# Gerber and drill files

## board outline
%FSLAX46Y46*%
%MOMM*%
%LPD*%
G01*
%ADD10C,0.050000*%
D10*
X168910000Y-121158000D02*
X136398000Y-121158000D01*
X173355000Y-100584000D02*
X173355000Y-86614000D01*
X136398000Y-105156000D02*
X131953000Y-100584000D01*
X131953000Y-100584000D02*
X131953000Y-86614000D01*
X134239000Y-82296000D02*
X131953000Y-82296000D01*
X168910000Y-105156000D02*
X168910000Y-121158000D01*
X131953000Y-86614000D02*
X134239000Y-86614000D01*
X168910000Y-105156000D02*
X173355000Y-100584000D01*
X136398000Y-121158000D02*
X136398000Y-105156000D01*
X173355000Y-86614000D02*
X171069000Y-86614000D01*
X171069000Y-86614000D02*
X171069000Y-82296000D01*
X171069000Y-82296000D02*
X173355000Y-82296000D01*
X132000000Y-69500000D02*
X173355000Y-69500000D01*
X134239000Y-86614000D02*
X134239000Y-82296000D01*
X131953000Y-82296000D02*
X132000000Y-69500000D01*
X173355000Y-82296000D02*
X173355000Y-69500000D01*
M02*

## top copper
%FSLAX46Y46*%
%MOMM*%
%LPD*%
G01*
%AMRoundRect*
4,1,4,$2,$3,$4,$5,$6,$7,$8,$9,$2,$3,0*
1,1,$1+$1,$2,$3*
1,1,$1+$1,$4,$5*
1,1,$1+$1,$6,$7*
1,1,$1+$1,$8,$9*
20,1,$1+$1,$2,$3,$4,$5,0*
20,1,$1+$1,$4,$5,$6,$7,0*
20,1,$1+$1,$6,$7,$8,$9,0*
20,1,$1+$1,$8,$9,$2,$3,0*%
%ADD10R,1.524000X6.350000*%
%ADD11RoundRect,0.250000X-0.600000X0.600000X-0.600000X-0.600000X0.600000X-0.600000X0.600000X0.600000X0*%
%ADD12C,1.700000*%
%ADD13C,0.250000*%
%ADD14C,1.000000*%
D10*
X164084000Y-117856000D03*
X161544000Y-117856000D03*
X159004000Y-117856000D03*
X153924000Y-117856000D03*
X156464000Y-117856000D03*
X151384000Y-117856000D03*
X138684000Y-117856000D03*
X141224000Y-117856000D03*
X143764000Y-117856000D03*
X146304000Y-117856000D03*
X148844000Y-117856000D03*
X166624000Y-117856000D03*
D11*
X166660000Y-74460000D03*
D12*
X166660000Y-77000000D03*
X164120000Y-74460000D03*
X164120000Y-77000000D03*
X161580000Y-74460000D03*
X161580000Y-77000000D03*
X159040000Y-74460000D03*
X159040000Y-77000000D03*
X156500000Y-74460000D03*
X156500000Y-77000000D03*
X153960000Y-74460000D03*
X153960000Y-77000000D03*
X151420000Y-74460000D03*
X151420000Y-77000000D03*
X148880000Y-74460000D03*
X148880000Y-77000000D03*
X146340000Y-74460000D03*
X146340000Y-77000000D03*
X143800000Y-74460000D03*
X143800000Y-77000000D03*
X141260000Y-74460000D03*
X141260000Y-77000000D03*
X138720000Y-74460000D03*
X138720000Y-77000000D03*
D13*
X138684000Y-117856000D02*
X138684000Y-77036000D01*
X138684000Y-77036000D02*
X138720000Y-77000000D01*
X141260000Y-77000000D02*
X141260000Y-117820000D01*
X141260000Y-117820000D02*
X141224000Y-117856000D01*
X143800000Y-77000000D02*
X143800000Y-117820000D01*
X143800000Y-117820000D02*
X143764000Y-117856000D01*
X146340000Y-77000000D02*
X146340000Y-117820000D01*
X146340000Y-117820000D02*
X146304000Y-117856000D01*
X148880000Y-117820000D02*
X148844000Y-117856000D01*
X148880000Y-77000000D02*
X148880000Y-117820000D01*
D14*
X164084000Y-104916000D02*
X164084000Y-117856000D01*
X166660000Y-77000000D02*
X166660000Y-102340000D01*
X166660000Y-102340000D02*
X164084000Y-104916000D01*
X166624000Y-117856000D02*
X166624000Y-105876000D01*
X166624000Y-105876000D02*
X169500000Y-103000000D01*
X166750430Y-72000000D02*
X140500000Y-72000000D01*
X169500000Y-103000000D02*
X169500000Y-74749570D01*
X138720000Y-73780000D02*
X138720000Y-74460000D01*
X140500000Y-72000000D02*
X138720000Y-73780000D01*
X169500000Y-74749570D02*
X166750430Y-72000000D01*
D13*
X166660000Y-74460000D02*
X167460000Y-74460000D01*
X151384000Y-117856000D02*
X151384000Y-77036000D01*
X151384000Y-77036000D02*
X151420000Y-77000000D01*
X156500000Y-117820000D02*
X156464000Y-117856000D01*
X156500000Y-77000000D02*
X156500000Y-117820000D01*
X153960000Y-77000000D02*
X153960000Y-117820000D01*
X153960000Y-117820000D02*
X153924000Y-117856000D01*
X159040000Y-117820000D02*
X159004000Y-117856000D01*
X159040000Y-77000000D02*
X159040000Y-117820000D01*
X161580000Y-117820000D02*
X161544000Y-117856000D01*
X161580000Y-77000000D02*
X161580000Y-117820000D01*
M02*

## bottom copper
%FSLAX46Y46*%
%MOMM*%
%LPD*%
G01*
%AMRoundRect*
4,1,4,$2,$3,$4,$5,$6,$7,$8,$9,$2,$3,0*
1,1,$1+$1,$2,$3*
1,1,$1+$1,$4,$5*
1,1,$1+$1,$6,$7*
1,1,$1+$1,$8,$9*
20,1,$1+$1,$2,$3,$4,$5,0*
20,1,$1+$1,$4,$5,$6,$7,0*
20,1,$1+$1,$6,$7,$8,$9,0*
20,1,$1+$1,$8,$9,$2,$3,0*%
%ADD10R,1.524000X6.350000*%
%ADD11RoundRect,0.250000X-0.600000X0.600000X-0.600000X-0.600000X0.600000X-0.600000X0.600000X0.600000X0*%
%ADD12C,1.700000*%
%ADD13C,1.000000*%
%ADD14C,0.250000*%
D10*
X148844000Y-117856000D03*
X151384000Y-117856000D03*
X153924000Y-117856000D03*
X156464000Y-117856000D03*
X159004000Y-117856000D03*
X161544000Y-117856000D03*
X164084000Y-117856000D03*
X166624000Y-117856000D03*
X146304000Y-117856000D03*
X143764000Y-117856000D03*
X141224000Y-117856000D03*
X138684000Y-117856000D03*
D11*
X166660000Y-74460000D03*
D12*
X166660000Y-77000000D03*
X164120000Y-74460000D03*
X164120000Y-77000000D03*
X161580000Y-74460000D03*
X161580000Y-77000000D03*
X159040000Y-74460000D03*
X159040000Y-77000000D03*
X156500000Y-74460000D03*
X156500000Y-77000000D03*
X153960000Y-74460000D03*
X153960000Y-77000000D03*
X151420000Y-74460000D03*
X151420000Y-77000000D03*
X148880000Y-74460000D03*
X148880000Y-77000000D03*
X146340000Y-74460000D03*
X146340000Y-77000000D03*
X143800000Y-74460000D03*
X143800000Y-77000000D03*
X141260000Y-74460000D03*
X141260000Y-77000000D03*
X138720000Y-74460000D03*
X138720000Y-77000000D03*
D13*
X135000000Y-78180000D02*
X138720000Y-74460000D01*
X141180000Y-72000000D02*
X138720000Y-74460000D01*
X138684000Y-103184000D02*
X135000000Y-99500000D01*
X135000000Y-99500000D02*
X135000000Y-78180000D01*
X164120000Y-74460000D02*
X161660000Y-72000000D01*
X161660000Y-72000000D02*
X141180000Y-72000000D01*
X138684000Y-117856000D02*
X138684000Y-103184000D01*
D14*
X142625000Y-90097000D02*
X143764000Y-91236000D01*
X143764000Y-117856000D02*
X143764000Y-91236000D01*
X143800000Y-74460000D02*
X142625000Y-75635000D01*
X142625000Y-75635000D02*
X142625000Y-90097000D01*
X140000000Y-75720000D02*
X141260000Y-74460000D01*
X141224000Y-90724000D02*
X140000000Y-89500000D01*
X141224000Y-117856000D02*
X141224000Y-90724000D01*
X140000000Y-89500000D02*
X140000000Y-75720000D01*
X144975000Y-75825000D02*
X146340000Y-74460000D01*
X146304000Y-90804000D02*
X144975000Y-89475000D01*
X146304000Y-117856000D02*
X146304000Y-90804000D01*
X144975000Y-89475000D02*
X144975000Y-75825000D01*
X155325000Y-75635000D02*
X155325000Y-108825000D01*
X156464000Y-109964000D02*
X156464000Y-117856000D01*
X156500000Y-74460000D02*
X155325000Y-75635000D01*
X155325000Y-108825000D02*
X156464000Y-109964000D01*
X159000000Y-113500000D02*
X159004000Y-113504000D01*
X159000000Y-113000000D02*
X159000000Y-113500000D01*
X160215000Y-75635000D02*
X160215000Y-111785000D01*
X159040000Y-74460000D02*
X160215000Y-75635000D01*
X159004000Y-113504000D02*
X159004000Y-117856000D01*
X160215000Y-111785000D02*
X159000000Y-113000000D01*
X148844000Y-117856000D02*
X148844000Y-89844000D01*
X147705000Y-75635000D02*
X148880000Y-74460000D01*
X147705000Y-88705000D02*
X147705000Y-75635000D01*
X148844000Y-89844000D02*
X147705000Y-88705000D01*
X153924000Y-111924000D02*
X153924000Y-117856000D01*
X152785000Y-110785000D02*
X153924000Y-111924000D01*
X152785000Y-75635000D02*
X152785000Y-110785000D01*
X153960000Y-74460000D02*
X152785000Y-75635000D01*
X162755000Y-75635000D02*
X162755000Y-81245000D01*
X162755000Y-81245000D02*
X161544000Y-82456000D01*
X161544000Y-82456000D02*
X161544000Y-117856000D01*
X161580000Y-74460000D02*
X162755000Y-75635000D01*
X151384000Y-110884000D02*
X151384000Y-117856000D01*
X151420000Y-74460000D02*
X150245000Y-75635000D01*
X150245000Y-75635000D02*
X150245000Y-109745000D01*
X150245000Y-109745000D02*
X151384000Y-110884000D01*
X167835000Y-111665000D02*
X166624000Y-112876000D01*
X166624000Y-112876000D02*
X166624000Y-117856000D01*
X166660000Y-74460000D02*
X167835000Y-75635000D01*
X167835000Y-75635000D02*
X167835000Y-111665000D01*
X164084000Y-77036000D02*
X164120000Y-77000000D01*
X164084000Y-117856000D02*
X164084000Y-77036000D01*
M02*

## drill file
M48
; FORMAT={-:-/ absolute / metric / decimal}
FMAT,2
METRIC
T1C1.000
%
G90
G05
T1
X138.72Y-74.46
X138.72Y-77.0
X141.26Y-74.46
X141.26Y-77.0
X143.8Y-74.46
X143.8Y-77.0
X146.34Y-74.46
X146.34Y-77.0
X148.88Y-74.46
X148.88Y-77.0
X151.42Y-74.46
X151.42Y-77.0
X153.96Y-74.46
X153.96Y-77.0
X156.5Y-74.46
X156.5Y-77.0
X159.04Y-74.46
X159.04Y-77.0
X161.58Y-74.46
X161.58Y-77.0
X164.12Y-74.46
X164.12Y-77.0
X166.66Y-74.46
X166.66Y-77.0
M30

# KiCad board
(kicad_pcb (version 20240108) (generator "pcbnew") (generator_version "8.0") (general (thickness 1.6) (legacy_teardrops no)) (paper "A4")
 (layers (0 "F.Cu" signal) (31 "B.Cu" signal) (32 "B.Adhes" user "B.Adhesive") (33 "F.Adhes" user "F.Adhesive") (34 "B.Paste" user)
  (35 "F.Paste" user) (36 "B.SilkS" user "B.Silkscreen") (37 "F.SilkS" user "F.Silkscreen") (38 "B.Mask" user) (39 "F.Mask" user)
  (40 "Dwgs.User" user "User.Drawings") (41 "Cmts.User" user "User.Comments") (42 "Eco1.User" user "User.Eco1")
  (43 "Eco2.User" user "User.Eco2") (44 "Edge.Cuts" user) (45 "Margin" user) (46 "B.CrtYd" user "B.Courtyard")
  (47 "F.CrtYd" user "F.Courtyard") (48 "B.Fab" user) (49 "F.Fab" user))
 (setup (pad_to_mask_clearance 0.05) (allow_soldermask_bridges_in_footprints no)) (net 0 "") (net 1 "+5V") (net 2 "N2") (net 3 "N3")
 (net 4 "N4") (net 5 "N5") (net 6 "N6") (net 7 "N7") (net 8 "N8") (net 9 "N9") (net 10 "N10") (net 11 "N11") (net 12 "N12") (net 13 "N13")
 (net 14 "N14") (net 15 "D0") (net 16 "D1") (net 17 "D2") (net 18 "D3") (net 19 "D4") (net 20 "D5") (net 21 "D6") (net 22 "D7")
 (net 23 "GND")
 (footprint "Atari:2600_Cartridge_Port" (layer "F.Cu") (at 138.176 114.808)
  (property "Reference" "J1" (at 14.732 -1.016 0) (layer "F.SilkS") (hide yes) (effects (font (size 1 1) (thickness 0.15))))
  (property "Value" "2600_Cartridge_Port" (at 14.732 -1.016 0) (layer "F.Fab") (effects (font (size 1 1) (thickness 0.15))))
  (pad "+5V" connect rect (at 25.908 3.048) (size 1.524 6.35) (layers "F.Cu" "F.Mask") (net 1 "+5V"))
  (pad "A0" connect rect (at 10.668 3.048) (size 1.524 6.35) (layers "B.Cu" "B.Mask") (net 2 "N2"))
  (pad "A1" connect rect (at 13.208 3.048) (size 1.524 6.35) (layers "B.Cu" "B.Mask") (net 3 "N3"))
  (pad "A2" connect rect (at 15.748 3.048) (size 1.524 6.35) (layers "B.Cu" "B.Mask") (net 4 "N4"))
  (pad "A3" connect rect (at 18.288 3.048) (size 1.524 6.35) (layers "B.Cu" "B.Mask") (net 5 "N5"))
  (pad "A4" connect rect (at 20.828 3.048) (size 1.524 6.35) (layers "B.Cu" "B.Mask") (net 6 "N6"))
  (pad "A5" connect rect (at 23.368 3.048) (size 1.524 6.35) (layers "B.Cu" "B.Mask") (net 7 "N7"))
  (pad "A6" connect rect (at 25.908 3.048) (size 1.524 6.35) (layers "B.Cu" "B.Mask") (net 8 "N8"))
  (pad "A7" connect rect (at 28.448 3.048) (size 1.524 6.35) (layers "B.Cu" "B.Mask") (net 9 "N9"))
  (pad "A8" connect rect (at 23.368 3.048) (size 1.524 6.35) (layers "F.Cu" "F.Mask") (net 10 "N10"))
  (pad "A9" connect rect (at 20.828 3.048) (size 1.524 6.35) (layers "F.Cu" "F.Mask") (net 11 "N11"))
  (pad "A10" connect rect (at 15.748 3.048) (size 1.524 6.35) (layers "F.Cu" "F.Mask") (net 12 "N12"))
  (pad "A11" connect rect (at 18.288 3.048) (size 1.524 6.35) (layers "F.Cu" "F.Mask") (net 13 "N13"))
  (pad "A12" connect rect (at 13.208 3.048) (size 1.524 6.35) (layers "F.Cu" "F.Mask") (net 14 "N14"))
  (pad "D0" connect rect (at 8.128 3.048) (size 1.524 6.35) (layers "B.Cu" "B.Mask") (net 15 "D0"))
  (pad "D1" connect rect (at 5.588 3.048) (size 1.524 6.35) (layers "B.Cu" "B.Mask") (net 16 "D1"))
  (pad "D2" connect rect (at 3.048 3.048) (size 1.524 6.35) (layers "B.Cu" "B.Mask") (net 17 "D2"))
  (pad "D3" connect rect (at 0.508 3.048) (size 1.524 6.35) (layers "F.Cu" "F.Mask") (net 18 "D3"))
  (pad "D4" connect rect (at 3.048 3.048) (size 1.524 6.35) (layers "F.Cu" "F.Mask") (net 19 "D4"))
  (pad "D5" connect rect (at 5.588 3.048) (size 1.524 6.35) (layers "F.Cu" "F.Mask") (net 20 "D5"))
  (pad "D6" connect rect (at 8.128 3.048) (size 1.524 6.35) (layers "F.Cu" "F.Mask") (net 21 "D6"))
  (pad "D7" connect rect (at 10.668 3.048) (size 1.524 6.35) (layers "F.Cu" "F.Mask") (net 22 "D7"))
  (pad "GND" connect rect (at 0.508 3.048) (size 1.524 6.35) (layers "B.Cu" "B.Mask") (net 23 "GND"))
  (pad "SGND" connect rect (at 28.448 3.048) (size 1.524 6.35) (layers "F.Cu" "F.Mask") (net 23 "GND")))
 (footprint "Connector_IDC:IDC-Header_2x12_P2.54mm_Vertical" (layer "F.Cu") (at 166.66 74.46 -90)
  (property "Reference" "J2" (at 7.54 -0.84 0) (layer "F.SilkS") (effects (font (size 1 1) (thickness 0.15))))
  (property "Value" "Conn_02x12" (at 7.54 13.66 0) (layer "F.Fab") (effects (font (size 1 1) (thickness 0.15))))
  (pad "1" thru_hole roundrect (at 0 0 270) (size 1.7 1.7) (drill 1) (layers "*.Cu" "*.Mask") (remove_unused_layers no)
   (roundrect_rratio 0.147059) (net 9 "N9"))
  (pad "2" thru_hole circle (at 2.54 0 270) (size 1.7 1.7) (drill 1) (layers "*.Cu" "*.Mask") (remove_unused_layers no) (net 1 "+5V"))
  (pad "3" thru_hole circle (at 0 2.54 270) (size 1.7 1.7) (drill 1) (layers "*.Cu" "*.Mask") (remove_unused_layers no) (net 23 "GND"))
  (pad "4" thru_hole circle (at 2.54 2.54 270) (size 1.7 1.7) (drill 1) (layers "*.Cu" "*.Mask") (remove_unused_layers no) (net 8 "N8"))
  (pad "5" thru_hole circle (at 0 5.08 270) (size 1.7 1.7) (drill 1) (layers "*.Cu" "*.Mask") (remove_unused_layers no) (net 7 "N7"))
  (pad "6" thru_hole circle (at 2.54 5.08 270) (size 1.7 1.7) (drill 1) (layers "*.Cu" "*.Mask") (remove_unused_layers no) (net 10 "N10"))
  (pad "7" thru_hole circle (at 0 7.62 270) (size 1.7 1.7) (drill 1) (layers "*.Cu" "*.Mask") (remove_unused_layers no) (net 6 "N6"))
  (pad "8" thru_hole circle (at 2.54 7.62 270) (size 1.7 1.7) (drill 1) (layers "*.Cu" "*.Mask") (remove_unused_layers no) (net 11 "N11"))
  (pad "9" thru_hole circle (at 0 10.16 270) (size 1.7 1.7) (drill 1) (layers "*.Cu" "*.Mask") (remove_unused_layers no) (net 5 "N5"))
  (pad "10" thru_hole circle (at 2.54 10.16 270) (size 1.7 1.7) (drill 1) (layers "*.Cu" "*.Mask") (remove_unused_layers no) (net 13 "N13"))
  (pad "11" thru_hole circle (at 0 12.7 270) (size 1.7 1.7) (drill 1) (layers "*.Cu" "*.Mask") (remove_unused_layers no) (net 4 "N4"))
  (pad "12" thru_hole circle (at 2.54 12.7 270) (size 1.7 1.7) (drill 1) (layers "*.Cu" "*.Mask") (remove_unused_layers no) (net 12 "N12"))
  (pad "13" thru_hole circle (at 0 15.24 270) (size 1.7 1.7) (drill 1) (layers "*.Cu" "*.Mask") (remove_unused_layers no) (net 3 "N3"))
  (pad "14" thru_hole circle (at 2.54 15.24 270) (size 1.7 1.7) (drill 1) (layers "*.Cu" "*.Mask") (remove_unused_layers no) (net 14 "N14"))
  (pad "15" thru_hole circle (at 0 17.78 270) (size 1.7 1.7) (drill 1) (layers "*.Cu" "*.Mask") (remove_unused_layers no) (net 2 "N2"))
  (pad "16" thru_hole circle (at 2.54 17.78 270) (size 1.7 1.7) (drill 1) (layers "*.Cu" "*.Mask") (remove_unused_layers no) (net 22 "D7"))
  (pad "17" thru_hole circle (at 0 20.32 270) (size 1.7 1.7) (drill 1) (layers "*.Cu" "*.Mask") (remove_unused_layers no) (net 15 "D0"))
  (pad "18" thru_hole circle (at 2.54 20.32 270) (size 1.7 1.7) (drill 1) (layers "*.Cu" "*.Mask") (remove_unused_layers no) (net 21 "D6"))
  (pad "19" thru_hole circle (at 0 22.86 270) (size 1.7 1.7) (drill 1) (layers "*.Cu" "*.Mask") (remove_unused_layers no) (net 16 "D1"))
  (pad "20" thru_hole circle (at 2.54 22.86 270) (size 1.7 1.7) (drill 1) (layers "*.Cu" "*.Mask") (remove_unused_layers no) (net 20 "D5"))
  (pad "21" thru_hole circle (at 0 25.4 270) (size 1.7 1.7) (drill 1) (layers "*.Cu" "*.Mask") (remove_unused_layers no) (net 17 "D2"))
  (pad "22" thru_hole circle (at 2.54 25.4 270) (size 1.7 1.7) (drill 1) (layers "*.Cu" "*.Mask") (remove_unused_layers no) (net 19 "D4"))
  (pad "23" thru_hole circle (at 0 27.94 270) (size 1.7 1.7) (drill 1) (layers "*.Cu" "*.Mask") (remove_unused_layers no) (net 23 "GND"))
  (pad "24" thru_hole circle (at 2.54 27.94 270) (size 1.7 1.7) (drill 1) (layers "*.Cu" "*.Mask") (remove_unused_layers no) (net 18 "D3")))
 (gr_line (start 168.91 121.158) (end 136.398 121.158) (stroke (width 0.05) (type solid)) (layer "Edge.Cuts"))
 (gr_line (start 173.355 100.584) (end 173.355 86.614) (stroke (width 0.05) (type solid)) (layer "Edge.Cuts"))
 (gr_line (start 136.398 105.156) (end 131.953 100.584) (stroke (width 0.05) (type solid)) (layer "Edge.Cuts"))
 (gr_line (start 131.953 100.584) (end 131.953 86.614) (stroke (width 0.05) (type solid)) (layer "Edge.Cuts"))
 (gr_line (start 134.239 82.296) (end 131.953 82.296) (stroke (width 0.05) (type solid)) (layer "Edge.Cuts"))
 (gr_line (start 168.91 105.156) (end 168.91 121.158) (stroke (width 0.05) (type solid)) (layer "Edge.Cuts"))
 (gr_line (start 131.953 86.614) (end 134.239 86.614) (stroke (width 0.05) (type solid)) (layer "Edge.Cuts"))
 (gr_line (start 168.91 105.156) (end 173.355 100.584) (stroke (width 0.05) (type solid)) (layer "Edge.Cuts"))
 (gr_line (start 136.398 121.158) (end 136.398 105.156) (stroke (width 0.05) (type solid)) (layer "Edge.Cuts"))
 (gr_line (start 173.355 86.614) (end 171.069 86.614) (stroke (width 0.05) (type solid)) (layer "Edge.Cuts"))
 (gr_line (start 171.069 86.614) (end 171.069 82.296) (stroke (width 0.05) (type solid)) (layer "Edge.Cuts"))
 (gr_line (start 171.069 82.296) (end 173.355 82.296) (stroke (width 0.05) (type solid)) (layer "Edge.Cuts"))
 (gr_line (start 132 69.5) (end 173.355 69.5) (stroke (width 0.05) (type solid)) (layer "Edge.Cuts"))
 (gr_line (start 134.239 86.614) (end 134.239 82.296) (stroke (width 0.05) (type solid)) (layer "Edge.Cuts"))
 (gr_line (start 131.953 82.296) (end 132 69.5) (stroke (width 0.05) (type solid)) (layer "Edge.Cuts"))
 (gr_line (start 173.355 82.296) (end 173.355 69.5) (stroke (width 0.05) (type solid)) (layer "Edge.Cuts"))
 (segment (start 138.684 117.856) (end 138.684 77.036) (width 0.25) (layer "F.Cu") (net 18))
 (segment (start 138.684 77.036) (end 138.72 77) (width 0.25) (layer "F.Cu") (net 18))
 (segment (start 141.26 77) (end 141.26 117.82) (width 0.25) (layer "F.Cu") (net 19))
 (segment (start 141.26 117.82) (end 141.224 117.856) (width 0.25) (layer "F.Cu") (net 19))
 (segment (start 143.8 77) (end 143.8 117.82) (width 0.25) (layer "F.Cu") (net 20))
 (segment (start 143.8 117.82) (end 143.764 117.856) (width 0.25) (layer "F.Cu") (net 20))
 (segment (start 146.34 77) (end 146.34 117.82) (width 0.25) (layer "F.Cu") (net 21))
 (segment (start 146.34 117.82) (end 146.304 117.856) (width 0.25) (layer "F.Cu") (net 21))
 (segment (start 148.88 117.82) (end 148.844 117.856) (width 0.25) (layer "F.Cu") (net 22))
 (segment (start 148.88 77) (end 148.88 117.82) (width 0.25) (layer "F.Cu") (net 22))
 (segment (start 164.084 104.916) (end 164.084 117.856) (width 1) (layer "F.Cu") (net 1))
 (segment (start 166.66 77) (end 166.66 102.34) (width 1) (layer "F.Cu") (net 1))
 (segment (start 166.66 102.34) (end 164.084 104.916) (width 1) (layer "F.Cu") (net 1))
 (segment (start 166.624 117.856) (end 166.624 105.876) (width 1) (layer "F.Cu") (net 23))
 (segment (start 166.624 105.876) (end 169.5 103) (width 1) (layer "F.Cu") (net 23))
 (segment (start 166.75043 72) (end 140.5 72) (width 1) (layer "F.Cu") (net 23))
 (segment (start 169.5 103) (end 169.5 74.74957) (width 1) (layer "F.Cu") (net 23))
 (segment (start 138.72 73.78) (end 138.72 74.46) (width 1) (layer "F.Cu") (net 23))
 (segment (start 140.5 72) (end 138.72 73.78) (width 1) (layer "F.Cu") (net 23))
 (segment (start 169.5 74.74957) (end 166.75043 72) (width 1) (layer "F.Cu") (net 23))
 (segment (start 135 78.18) (end 138.72 74.46) (width 1) (layer "B.Cu") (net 23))
 (segment (start 141.18 72) (end 138.72 74.46) (width 1) (layer "B.Cu") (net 23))
 (segment (start 138.684 103.184) (end 135 99.5) (width 1) (layer "B.Cu") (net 23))
 (segment (start 135 99.5) (end 135 78.18) (width 1) (layer "B.Cu") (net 23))
 (segment (start 164.12 74.46) (end 161.66 72) (width 1) (layer "B.Cu") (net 23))
 (segment (start 161.66 72) (end 141.18 72) (width 1) (layer "B.Cu") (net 23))
 (segment (start 138.684 117.856) (end 138.684 103.184) (width 1) (layer "B.Cu") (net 23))
 (segment (start 142.625 90.097) (end 143.764 91.236) (width 0.25) (layer "B.Cu") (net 16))
 (segment (start 143.764 117.856) (end 143.764 91.236) (width 0.25) (layer "B.Cu") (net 16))
 (segment (start 143.8 74.46) (end 142.625 75.635) (width 0.25) (layer "B.Cu") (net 16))
 (segment (start 142.625 75.635) (end 142.625 90.097) (width 0.25) (layer "B.Cu") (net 16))
 (segment (start 140 75.72) (end 141.26 74.46) (width 0.25) (layer "B.Cu") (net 17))
 (segment (start 141.224 90.724) (end 140 89.5) (width 0.25) (layer "B.Cu") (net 17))
 (segment (start 141.224 117.856) (end 141.224 90.724) (width 0.25) (layer "B.Cu") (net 17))
 (segment (start 140 89.5) (end 140 75.72) (width 0.25) (layer "B.Cu") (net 17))
 (segment (start 144.975 75.825) (end 146.34 74.46) (width 0.25) (layer "B.Cu") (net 15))
 (segment (start 146.304 90.804) (end 144.975 89.475) (width 0.25) (layer "B.Cu") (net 15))
 (segment (start 146.304 117.856) (end 146.304 90.804) (width 0.25) (layer "B.Cu") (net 15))
 (segment (start 144.975 89.475) (end 144.975 75.825) (width 0.25) (layer "B.Cu") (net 15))
 (segment (start 155.325 75.635) (end 155.325 108.825) (width 0.25) (layer "B.Cu") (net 5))
 (segment (start 156.464 109.964) (end 156.464 117.856) (width 0.25) (layer "B.Cu") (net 5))
 (segment (start 156.5 74.46) (end 155.325 75.635) (width 0.25) (layer "B.Cu") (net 5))
 (segment (start 155.325 108.825) (end 156.464 109.964) (width 0.25) (layer "B.Cu") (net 5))
 (segment (start 159 113.5) (end 159.004 113.504) (width 0.25) (layer "B.Cu") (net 6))
 (segment (start 159 113) (end 159 113.5) (width 0.25) (layer "B.Cu") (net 6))
 (segment (start 160.215 75.635) (end 160.215 111.785) (width 0.25) (layer "B.Cu") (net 6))
 (segment (start 159.04 74.46) (end 160.215 75.635) (width 0.25) (layer "B.Cu") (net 6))
 (segment (start 159.004 113.504) (end 159.004 117.856) (width 0.25) (layer "B.Cu") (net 6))
 (segment (start 160.215 111.785) (end 159 113) (width 0.25) (layer "B.Cu") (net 6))
 (segment (start 148.844 117.856) (end 148.844 89.844) (width 0.25) (layer "B.Cu") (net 2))
 (segment (start 147.705 75.635) (end 148.88 74.46) (width 0.25) (layer "B.Cu") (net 2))
 (segment (start 147.705 88.705) (end 147.705 75.635) (width 0.25) (layer "B.Cu") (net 2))
 (segment (start 148.844 89.844) (end 147.705 88.705) (width 0.25) (layer "B.Cu") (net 2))
 (segment (start 153.924 111.924) (end 153.924 117.856) (width 0.25) (layer "B.Cu") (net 4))
 (segment (start 152.785 110.785) (end 153.924 111.924) (width 0.25) (layer "B.Cu") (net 4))
 (segment (start 152.785 75.635) (end 152.785 110.785) (width 0.25) (layer "B.Cu") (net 4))
 (segment (start 153.96 74.46) (end 152.785 75.635) (width 0.25) (layer "B.Cu") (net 4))
 (segment (start 162.755 75.635) (end 162.755 81.245) (width 0.25) (layer "B.Cu") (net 7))
 (segment (start 162.755 81.245) (end 161.544 82.456) (width 0.25) (layer "B.Cu") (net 7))
 (segment (start 161.544 82.456) (end 161.544 117.856) (width 0.25) (layer "B.Cu") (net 7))
 (segment (start 161.58 74.46) (end 162.755 75.635) (width 0.25) (layer "B.Cu") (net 7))
 (segment (start 151.384 110.884) (end 151.384 117.856) (width 0.25) (layer "B.Cu") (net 3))
 (segment (start 151.42 74.46) (end 150.245 75.635) (width 0.25) (layer "B.Cu") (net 3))
 (segment (start 150.245 75.635) (end 150.245 109.745) (width 0.25) (layer "B.Cu") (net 3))
 (segment (start 150.245 109.745) (end 151.384 110.884) (width 0.25) (layer "B.Cu") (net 3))
 (segment (start 166.66 74.46) (end 167.46 74.46) (width 0.25) (layer "F.Cu") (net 9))
 (segment (start 167.835 111.665) (end 166.624 112.876) (width 0.25) (layer "B.Cu") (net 9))
 (segment (start 166.624 112.876) (end 166.624 117.856) (width 0.25) (layer "B.Cu") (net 9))
 (segment (start 166.66 74.46) (end 167.835 75.635) (width 0.25) (layer "B.Cu") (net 9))
 (segment (start 167.835 75.635) (end 167.835 111.665) (width 0.25) (layer "B.Cu") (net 9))
 (segment (start 151.384 117.856) (end 151.384 77.036) (width 0.25) (layer "F.Cu") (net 14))
 (segment (start 151.384 77.036) (end 151.42 77) (width 0.25) (layer "F.Cu") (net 14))
 (segment (start 156.5 117.82) (end 156.464 117.856) (width 0.25) (layer "F.Cu") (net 13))
 (segment (start 156.5 77) (end 156.5 117.82) (width 0.25) (layer "F.Cu") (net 13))
 (segment (start 153.96 77) (end 153.96 117.82) (width 0.25) (layer "F.Cu") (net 12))
 (segment (start 153.96 117.82) (end 153.924 117.856) (width 0.25) (layer "F.Cu") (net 12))
 (segment (start 159.04 117.82) (end 159.004 117.856) (width 0.25) (layer "F.Cu") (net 11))
 (segment (start 159.04 77) (end 159.04 117.82) (width 0.25) (layer "F.Cu") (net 11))
 (segment (start 161.58 117.82) (end 161.544 117.856) (width 0.25) (layer "F.Cu") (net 10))
 (segment (start 161.58 77) (end 161.58 117.82) (width 0.25) (layer "F.Cu") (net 10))
 (segment (start 164.084 77.036) (end 164.12 77) (width 0.25) (layer "B.Cu") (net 8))
 (segment (start 164.084 117.856) (end 164.084 77.036) (width 0.25) (layer "B.Cu") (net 8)))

